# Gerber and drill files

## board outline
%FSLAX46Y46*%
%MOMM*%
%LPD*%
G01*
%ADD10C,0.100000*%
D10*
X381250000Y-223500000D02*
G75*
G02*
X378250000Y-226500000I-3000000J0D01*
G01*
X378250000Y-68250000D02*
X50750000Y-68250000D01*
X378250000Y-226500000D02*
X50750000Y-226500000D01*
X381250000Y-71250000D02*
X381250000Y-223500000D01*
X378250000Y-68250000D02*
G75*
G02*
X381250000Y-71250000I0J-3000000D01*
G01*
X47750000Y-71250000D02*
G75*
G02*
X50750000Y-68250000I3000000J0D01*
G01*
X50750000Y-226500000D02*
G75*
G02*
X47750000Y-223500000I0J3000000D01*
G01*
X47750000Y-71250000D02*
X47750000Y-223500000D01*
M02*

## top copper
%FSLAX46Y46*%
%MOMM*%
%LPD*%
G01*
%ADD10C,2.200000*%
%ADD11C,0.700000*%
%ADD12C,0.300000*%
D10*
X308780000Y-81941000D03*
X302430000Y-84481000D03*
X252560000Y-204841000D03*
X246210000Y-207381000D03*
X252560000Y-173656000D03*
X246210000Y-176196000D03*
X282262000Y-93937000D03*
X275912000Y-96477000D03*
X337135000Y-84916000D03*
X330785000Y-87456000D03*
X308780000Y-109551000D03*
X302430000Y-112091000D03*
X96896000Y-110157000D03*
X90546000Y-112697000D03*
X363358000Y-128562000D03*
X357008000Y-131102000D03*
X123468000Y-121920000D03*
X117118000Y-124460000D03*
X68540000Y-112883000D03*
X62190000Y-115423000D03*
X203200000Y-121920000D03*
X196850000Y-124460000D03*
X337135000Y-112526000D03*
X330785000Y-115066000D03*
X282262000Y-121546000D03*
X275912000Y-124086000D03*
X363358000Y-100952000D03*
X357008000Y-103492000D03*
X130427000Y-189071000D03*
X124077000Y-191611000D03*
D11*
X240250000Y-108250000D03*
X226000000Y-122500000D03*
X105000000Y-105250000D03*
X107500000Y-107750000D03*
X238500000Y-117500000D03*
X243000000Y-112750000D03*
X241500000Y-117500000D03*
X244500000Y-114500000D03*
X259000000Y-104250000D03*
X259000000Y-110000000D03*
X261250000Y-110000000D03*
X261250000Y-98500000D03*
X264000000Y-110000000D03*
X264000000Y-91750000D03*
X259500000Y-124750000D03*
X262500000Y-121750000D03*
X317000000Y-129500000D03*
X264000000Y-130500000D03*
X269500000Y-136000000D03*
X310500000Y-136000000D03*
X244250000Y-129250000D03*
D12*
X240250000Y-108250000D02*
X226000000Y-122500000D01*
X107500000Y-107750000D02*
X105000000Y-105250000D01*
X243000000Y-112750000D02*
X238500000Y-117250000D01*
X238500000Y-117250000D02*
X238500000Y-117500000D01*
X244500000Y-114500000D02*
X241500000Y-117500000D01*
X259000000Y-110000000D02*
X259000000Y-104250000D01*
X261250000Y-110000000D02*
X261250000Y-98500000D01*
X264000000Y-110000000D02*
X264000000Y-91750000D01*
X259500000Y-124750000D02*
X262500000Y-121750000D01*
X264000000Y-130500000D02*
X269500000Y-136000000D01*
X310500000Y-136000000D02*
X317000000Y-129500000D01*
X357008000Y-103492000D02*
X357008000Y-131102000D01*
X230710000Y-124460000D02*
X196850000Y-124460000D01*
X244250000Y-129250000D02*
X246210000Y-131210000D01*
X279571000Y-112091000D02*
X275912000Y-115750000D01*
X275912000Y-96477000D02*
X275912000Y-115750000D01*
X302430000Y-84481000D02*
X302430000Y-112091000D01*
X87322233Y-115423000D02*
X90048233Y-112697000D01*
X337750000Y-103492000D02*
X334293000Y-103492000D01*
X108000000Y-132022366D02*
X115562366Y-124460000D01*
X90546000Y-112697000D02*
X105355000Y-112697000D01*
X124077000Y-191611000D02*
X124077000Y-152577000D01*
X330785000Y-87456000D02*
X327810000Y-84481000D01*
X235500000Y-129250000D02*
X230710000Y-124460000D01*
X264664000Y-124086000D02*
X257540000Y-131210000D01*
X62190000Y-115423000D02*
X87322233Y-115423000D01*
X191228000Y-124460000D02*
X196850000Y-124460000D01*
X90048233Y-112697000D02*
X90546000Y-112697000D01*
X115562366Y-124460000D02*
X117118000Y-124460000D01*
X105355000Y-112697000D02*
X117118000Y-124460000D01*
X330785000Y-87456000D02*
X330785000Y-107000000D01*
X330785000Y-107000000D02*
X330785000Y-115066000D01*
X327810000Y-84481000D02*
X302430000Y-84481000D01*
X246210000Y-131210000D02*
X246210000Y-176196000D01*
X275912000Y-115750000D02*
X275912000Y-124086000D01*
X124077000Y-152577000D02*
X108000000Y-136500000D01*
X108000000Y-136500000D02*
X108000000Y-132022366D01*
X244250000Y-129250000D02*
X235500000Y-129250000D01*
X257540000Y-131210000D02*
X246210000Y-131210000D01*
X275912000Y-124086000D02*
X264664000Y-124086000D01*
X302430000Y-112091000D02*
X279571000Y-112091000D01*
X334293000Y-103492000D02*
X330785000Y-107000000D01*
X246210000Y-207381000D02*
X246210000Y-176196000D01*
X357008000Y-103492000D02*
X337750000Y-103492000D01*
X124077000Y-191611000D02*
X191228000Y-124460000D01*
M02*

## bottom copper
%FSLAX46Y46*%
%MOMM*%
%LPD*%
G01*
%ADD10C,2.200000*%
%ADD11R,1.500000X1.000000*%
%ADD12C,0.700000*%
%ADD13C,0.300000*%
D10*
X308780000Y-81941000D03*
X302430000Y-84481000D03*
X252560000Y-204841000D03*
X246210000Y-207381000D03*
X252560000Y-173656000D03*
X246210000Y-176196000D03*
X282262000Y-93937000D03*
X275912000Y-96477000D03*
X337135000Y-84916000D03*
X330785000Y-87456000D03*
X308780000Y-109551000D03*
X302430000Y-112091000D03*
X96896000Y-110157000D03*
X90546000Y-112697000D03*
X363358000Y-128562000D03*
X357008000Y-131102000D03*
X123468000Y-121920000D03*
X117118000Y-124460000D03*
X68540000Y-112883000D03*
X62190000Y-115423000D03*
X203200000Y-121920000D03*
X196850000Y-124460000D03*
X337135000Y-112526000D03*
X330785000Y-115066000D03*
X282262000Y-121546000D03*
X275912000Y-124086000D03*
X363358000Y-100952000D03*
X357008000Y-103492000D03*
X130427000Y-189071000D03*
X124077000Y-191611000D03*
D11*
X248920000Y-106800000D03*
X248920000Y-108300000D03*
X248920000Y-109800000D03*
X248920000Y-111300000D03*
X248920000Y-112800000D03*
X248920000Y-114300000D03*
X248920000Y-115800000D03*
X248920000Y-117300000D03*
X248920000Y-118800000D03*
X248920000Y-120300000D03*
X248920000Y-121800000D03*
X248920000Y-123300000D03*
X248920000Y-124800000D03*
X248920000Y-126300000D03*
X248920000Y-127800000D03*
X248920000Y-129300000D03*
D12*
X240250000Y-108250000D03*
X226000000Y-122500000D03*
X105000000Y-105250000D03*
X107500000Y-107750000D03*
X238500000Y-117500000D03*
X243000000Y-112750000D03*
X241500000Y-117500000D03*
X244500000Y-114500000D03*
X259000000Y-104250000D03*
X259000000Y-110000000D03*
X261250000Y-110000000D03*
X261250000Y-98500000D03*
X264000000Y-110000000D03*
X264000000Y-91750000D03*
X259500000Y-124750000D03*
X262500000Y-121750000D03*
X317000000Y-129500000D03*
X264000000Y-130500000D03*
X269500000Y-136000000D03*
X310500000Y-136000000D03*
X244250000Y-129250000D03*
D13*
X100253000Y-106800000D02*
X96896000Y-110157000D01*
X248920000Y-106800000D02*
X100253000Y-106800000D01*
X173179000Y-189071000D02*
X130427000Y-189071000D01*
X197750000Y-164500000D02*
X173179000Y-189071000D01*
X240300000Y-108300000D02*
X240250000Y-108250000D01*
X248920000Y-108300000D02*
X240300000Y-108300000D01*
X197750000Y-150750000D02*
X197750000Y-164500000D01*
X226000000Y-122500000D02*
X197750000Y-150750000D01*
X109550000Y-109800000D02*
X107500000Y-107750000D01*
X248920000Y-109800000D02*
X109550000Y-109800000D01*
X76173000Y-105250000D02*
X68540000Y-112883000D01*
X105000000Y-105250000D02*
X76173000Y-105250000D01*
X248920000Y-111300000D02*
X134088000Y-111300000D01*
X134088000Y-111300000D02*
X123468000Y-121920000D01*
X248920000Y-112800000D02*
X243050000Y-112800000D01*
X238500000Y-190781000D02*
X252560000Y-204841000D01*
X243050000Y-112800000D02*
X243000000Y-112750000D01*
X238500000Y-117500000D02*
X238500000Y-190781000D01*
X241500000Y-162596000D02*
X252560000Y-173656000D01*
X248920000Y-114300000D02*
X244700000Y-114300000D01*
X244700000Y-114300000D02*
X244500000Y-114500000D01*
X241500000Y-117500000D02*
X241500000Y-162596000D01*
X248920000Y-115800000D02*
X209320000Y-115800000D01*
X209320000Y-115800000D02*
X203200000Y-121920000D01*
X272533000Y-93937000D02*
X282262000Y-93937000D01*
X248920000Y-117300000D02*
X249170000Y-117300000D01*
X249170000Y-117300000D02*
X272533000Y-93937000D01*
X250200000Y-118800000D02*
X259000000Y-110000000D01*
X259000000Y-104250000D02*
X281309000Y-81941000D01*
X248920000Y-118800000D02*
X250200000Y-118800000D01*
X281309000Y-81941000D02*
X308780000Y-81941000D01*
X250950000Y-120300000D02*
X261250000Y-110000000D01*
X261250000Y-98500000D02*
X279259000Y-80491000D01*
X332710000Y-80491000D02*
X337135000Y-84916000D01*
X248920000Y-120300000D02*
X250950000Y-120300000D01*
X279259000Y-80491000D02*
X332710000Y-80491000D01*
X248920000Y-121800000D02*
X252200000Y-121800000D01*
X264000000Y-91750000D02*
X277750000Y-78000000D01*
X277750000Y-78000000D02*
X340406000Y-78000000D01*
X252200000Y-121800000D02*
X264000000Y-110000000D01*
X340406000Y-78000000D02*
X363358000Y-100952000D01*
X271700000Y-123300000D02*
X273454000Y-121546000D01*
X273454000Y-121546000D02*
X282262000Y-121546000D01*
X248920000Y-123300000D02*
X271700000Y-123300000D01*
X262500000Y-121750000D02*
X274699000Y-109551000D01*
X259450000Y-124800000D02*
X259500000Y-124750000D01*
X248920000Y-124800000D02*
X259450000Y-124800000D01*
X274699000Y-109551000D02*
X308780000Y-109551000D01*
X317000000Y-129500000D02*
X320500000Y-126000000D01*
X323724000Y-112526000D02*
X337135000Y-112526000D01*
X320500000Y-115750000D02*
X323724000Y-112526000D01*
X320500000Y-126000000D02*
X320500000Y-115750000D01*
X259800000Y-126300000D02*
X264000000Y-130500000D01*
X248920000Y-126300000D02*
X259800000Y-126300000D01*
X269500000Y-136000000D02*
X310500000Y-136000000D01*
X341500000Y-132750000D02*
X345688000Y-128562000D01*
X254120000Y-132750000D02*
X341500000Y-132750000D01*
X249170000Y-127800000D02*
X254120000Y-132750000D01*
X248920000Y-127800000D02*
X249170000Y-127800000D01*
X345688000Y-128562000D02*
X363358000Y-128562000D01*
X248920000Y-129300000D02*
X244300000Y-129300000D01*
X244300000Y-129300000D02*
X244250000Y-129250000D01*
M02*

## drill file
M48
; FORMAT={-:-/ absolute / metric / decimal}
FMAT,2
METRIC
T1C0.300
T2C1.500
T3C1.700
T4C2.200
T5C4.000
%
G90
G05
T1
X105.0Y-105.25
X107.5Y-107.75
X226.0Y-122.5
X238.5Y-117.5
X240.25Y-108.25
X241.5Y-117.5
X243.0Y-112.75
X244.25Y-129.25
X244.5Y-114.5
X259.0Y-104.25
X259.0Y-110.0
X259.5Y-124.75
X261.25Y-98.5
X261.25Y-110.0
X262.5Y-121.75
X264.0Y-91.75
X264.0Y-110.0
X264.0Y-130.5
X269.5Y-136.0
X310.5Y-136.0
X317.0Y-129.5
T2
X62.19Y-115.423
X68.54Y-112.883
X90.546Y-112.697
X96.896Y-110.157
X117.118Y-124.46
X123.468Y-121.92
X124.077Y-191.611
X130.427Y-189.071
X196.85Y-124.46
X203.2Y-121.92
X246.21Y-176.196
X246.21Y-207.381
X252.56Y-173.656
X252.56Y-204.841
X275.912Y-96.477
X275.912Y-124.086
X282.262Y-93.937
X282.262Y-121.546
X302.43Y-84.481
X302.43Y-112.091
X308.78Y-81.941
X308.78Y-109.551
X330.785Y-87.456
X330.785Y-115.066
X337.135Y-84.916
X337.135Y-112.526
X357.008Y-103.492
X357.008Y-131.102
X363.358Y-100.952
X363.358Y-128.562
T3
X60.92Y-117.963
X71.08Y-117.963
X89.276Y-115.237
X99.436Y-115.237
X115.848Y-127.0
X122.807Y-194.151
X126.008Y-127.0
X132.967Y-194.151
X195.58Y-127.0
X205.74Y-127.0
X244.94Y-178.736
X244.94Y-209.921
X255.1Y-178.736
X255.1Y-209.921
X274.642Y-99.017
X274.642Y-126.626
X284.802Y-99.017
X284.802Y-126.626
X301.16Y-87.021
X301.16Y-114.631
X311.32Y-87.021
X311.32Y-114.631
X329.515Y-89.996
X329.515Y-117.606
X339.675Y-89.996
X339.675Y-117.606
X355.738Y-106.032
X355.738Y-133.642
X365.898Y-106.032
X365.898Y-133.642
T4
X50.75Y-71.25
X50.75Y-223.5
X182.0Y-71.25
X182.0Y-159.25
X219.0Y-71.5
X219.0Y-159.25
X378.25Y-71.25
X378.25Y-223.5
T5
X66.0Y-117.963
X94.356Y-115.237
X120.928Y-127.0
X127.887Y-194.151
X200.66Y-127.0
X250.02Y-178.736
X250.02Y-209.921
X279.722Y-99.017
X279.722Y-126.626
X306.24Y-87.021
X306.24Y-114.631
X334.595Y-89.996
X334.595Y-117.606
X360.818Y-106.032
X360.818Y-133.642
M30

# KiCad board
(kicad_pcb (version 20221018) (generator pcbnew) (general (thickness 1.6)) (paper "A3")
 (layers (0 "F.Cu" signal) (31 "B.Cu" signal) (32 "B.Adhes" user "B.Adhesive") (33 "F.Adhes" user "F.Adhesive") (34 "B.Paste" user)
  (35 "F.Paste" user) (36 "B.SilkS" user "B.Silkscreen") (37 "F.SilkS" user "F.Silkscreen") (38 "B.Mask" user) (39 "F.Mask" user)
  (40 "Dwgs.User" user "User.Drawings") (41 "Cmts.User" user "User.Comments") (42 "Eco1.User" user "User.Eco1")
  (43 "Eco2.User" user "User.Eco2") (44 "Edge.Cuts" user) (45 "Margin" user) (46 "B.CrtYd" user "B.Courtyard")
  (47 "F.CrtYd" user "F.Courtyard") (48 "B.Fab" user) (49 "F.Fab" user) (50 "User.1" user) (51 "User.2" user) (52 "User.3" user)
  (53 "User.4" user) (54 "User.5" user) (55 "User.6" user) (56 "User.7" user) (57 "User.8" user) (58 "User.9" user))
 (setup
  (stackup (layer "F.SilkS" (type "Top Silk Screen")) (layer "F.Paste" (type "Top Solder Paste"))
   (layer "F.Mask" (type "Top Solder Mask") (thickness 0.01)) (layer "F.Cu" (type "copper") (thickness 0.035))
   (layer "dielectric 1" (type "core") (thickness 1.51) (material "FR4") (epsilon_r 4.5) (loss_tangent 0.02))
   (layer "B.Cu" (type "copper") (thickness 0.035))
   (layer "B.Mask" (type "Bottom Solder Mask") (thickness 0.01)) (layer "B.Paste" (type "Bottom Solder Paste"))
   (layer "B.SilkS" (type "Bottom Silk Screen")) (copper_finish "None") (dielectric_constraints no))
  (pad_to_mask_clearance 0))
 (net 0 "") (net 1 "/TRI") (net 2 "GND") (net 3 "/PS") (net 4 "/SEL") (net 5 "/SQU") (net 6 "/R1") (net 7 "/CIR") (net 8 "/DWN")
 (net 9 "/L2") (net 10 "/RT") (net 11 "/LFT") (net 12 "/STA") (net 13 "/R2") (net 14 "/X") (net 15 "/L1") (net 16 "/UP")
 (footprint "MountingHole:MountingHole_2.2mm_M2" (layer "F.Cu") (at 50.75 223.5)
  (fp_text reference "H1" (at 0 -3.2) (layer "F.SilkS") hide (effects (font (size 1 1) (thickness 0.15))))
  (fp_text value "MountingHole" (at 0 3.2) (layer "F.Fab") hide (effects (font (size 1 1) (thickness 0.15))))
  (pad "" np_thru_hole circle (at 0 0) (size 2.2 2.2) (drill 2.2) (layers "*.Cu" "*.Mask")))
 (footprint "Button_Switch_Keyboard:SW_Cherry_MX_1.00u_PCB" (layer "F.Cu") (at 308.78 81.941)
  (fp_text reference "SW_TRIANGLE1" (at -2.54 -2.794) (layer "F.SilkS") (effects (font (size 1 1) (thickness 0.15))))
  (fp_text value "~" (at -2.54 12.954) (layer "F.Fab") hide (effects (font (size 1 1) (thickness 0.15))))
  (pad "" np_thru_hole circle (at -7.62 5.08) (size 1.7 1.7) (drill 1.7) (layers "*.Cu" "*.Mask"))
  (pad "" np_thru_hole circle (at -2.54 5.08) (size 4 4) (drill 4) (layers "*.Cu" "*.Mask"))
  (pad "" np_thru_hole circle (at 2.54 5.08) (size 1.7 1.7) (drill 1.7) (layers "*.Cu" "*.Mask"))
  (pad "1" thru_hole circle (at 0 0) (size 2.2 2.2) (drill 1.5) (layers "*.Cu" "*.Mask") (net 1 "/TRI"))
  (pad "2" thru_hole circle (at -6.35 2.54) (size 2.2 2.2) (drill 1.5) (layers "*.Cu" "*.Mask") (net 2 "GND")))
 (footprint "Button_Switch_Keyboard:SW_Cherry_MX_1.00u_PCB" (layer "F.Cu") (at 252.56 204.841)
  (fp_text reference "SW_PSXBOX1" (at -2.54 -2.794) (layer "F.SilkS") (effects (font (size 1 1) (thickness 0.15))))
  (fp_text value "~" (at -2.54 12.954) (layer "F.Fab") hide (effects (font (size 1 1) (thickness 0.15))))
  (pad "" np_thru_hole circle (at -7.62 5.08) (size 1.7 1.7) (drill 1.7) (layers "*.Cu" "*.Mask"))
  (pad "" np_thru_hole circle (at -2.54 5.08) (size 4 4) (drill 4) (layers "*.Cu" "*.Mask"))
  (pad "" np_thru_hole circle (at 2.54 5.08) (size 1.7 1.7) (drill 1.7) (layers "*.Cu" "*.Mask"))
  (pad "1" thru_hole circle (at 0 0) (size 2.2 2.2) (drill 1.5) (layers "*.Cu" "*.Mask") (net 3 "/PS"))
  (pad "2" thru_hole circle (at -6.35 2.54) (size 2.2 2.2) (drill 1.5) (layers "*.Cu" "*.Mask") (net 2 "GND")))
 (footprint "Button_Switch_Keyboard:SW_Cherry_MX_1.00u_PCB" (layer "F.Cu") (at 252.56 173.656)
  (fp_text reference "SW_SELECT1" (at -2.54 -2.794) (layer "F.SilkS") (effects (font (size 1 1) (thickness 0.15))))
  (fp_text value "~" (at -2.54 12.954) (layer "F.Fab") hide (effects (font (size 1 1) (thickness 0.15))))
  (pad "" np_thru_hole circle (at -7.62 5.08) (size 1.7 1.7) (drill 1.7) (layers "*.Cu" "*.Mask"))
  (pad "" np_thru_hole circle (at -2.54 5.08) (size 4 4) (drill 4) (layers "*.Cu" "*.Mask"))
  (pad "" np_thru_hole circle (at 2.54 5.08) (size 1.7 1.7) (drill 1.7) (layers "*.Cu" "*.Mask"))
  (pad "1" thru_hole circle (at 0 0) (size 2.2 2.2) (drill 1.5) (layers "*.Cu" "*.Mask") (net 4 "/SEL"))
  (pad "2" thru_hole circle (at -6.35 2.54) (size 2.2 2.2) (drill 1.5) (layers "*.Cu" "*.Mask") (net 2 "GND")))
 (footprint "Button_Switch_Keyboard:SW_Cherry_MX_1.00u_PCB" (layer "F.Cu") (at 282.262 93.937)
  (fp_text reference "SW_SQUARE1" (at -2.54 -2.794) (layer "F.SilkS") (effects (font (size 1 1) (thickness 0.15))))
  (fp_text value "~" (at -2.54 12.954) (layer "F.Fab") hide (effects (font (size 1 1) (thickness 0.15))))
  (pad "" np_thru_hole circle (at -7.62 5.08) (size 1.7 1.7) (drill 1.7) (layers "*.Cu" "*.Mask"))
  (pad "" np_thru_hole circle (at -2.54 5.08) (size 4 4) (drill 4) (layers "*.Cu" "*.Mask"))
  (pad "" np_thru_hole circle (at 2.54 5.08) (size 1.7 1.7) (drill 1.7) (layers "*.Cu" "*.Mask"))
  (pad "1" thru_hole circle (at 0 0) (size 2.2 2.2) (drill 1.5) (layers "*.Cu" "*.Mask") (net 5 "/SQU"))
  (pad "2" thru_hole circle (at -6.35 2.54) (size 2.2 2.2) (drill 1.5) (layers "*.Cu" "*.Mask") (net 2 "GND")))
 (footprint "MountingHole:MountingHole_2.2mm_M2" (layer "F.Cu") (at 50.75 71.25)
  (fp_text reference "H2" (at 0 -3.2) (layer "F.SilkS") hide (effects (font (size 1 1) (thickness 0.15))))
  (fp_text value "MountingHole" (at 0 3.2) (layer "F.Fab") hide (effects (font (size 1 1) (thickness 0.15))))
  (pad "" np_thru_hole circle (at 0 0) (size 2.2 2.2) (drill 2.2) (layers "*.Cu" "*.Mask")))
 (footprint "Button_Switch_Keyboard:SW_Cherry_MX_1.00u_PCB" (layer "F.Cu") (at 337.135 84.916)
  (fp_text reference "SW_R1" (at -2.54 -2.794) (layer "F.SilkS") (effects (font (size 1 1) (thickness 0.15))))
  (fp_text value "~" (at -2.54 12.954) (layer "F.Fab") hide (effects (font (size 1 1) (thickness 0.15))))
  (pad "" np_thru_hole circle (at -7.62 5.08) (size 1.7 1.7) (drill 1.7) (layers "*.Cu" "*.Mask"))
  (pad "" np_thru_hole circle (at -2.54 5.08) (size 4 4) (drill 4) (layers "*.Cu" "*.Mask"))
  (pad "" np_thru_hole circle (at 2.54 5.08) (size 1.7 1.7) (drill 1.7) (layers "*.Cu" "*.Mask"))
  (pad "1" thru_hole circle (at 0 0) (size 2.2 2.2) (drill 1.5) (layers "*.Cu" "*.Mask") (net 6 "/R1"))
  (pad "2" thru_hole circle (at -6.35 2.54) (size 2.2 2.2) (drill 1.5) (layers "*.Cu" "*.Mask") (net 2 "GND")))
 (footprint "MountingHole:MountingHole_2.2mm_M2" (layer "F.Cu") (at 219 71.5)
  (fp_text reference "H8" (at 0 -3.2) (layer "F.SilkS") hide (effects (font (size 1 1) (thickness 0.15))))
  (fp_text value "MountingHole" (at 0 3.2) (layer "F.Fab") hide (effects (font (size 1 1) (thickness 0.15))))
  (pad "" np_thru_hole circle (at 0 0) (size 2.2 2.2) (drill 2.2) (layers "*.Cu" "*.Mask")))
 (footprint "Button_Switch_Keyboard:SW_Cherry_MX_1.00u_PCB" (layer "F.Cu") (at 308.78 109.551)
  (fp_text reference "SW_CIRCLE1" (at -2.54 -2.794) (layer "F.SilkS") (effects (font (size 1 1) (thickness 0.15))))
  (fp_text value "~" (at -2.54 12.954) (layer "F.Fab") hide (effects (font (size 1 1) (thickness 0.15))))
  (pad "" np_thru_hole circle (at -7.62 5.08) (size 1.7 1.7) (drill 1.7) (layers "*.Cu" "*.Mask"))
  (pad "" np_thru_hole circle (at -2.54 5.08) (size 4 4) (drill 4) (layers "*.Cu" "*.Mask"))
  (pad "" np_thru_hole circle (at 2.54 5.08) (size 1.7 1.7) (drill 1.7) (layers "*.Cu" "*.Mask"))
  (pad "1" thru_hole circle (at 0 0) (size 2.2 2.2) (drill 1.5) (layers "*.Cu" "*.Mask") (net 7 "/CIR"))
  (pad "2" thru_hole circle (at -6.35 2.54) (size 2.2 2.2) (drill 1.5) (layers "*.Cu" "*.Mask") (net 2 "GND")))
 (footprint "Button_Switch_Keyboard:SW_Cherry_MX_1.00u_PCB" (layer "F.Cu") (at 96.896 110.157)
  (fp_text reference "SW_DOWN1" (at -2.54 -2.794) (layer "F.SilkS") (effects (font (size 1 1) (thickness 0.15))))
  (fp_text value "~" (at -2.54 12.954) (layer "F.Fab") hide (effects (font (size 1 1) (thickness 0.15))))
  (pad "" np_thru_hole circle (at -7.62 5.08) (size 1.7 1.7) (drill 1.7) (layers "*.Cu" "*.Mask"))
  (pad "" np_thru_hole circle (at -2.54 5.08) (size 4 4) (drill 4) (layers "*.Cu" "*.Mask"))
  (pad "" np_thru_hole circle (at 2.54 5.08) (size 1.7 1.7) (drill 1.7) (layers "*.Cu" "*.Mask"))
  (pad "1" thru_hole circle (at 0 0) (size 2.2 2.2) (drill 1.5) (layers "*.Cu" "*.Mask") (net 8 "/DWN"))
  (pad "2" thru_hole circle (at -6.35 2.54) (size 2.2 2.2) (drill 1.5) (layers "*.Cu" "*.Mask") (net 2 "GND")))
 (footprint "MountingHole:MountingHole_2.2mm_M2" (layer "F.Cu") (at 219 159.25)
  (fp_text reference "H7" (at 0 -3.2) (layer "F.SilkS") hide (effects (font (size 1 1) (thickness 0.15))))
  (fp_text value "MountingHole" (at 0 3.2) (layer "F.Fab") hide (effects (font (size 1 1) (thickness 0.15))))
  (pad "" np_thru_hole circle (at 0 0) (size 2.2 2.2) (drill 2.2) (layers "*.Cu" "*.Mask")))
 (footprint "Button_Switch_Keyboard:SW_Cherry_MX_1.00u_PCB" (layer "F.Cu") (at 363.358 128.562)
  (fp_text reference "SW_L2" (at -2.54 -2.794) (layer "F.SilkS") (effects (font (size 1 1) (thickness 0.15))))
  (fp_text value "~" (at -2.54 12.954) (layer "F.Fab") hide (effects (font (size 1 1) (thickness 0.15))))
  (pad "" np_thru_hole circle (at -7.62 5.08) (size 1.7 1.7) (drill 1.7) (layers "*.Cu" "*.Mask"))
  (pad "" np_thru_hole circle (at -2.54 5.08) (size 4 4) (drill 4) (layers "*.Cu" "*.Mask"))
  (pad "" np_thru_hole circle (at 2.54 5.08) (size 1.7 1.7) (drill 1.7) (layers "*.Cu" "*.Mask"))
  (pad "1" thru_hole circle (at 0 0) (size 2.2 2.2) (drill 1.5) (layers "*.Cu" "*.Mask") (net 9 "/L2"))
  (pad "2" thru_hole circle (at -6.35 2.54) (size 2.2 2.2) (drill 1.5) (layers "*.Cu" "*.Mask") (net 2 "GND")))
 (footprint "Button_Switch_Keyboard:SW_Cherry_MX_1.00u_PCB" (layer "F.Cu") (at 123.468 121.92)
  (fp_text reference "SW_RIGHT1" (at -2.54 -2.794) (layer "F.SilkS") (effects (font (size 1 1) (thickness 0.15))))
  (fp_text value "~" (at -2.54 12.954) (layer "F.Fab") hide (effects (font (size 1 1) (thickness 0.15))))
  (pad "" np_thru_hole circle (at -7.62 5.08) (size 1.7 1.7) (drill 1.7) (layers "*.Cu" "*.Mask"))
  (pad "" np_thru_hole circle (at -2.54 5.08) (size 4 4) (drill 4) (layers "*.Cu" "*.Mask"))
  (pad "" np_thru_hole circle (at 2.54 5.08) (size 1.7 1.7) (drill 1.7) (layers "*.Cu" "*.Mask"))
  (pad "1" thru_hole circle (at 0 0) (size 2.2 2.2) (drill 1.5) (layers "*.Cu" "*.Mask") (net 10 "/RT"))
  (pad "2" thru_hole circle (at -6.35 2.54) (size 2.2 2.2) (drill 1.5) (layers "*.Cu" "*.Mask") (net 2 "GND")))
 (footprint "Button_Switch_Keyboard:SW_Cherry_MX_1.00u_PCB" (layer "F.Cu") (at 68.54 112.883)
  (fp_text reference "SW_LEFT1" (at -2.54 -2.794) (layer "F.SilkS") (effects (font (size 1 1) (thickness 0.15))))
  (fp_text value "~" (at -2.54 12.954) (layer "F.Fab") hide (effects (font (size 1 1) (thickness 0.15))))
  (pad "" np_thru_hole circle (at -7.62 5.08) (size 1.7 1.7) (drill 1.7) (layers "*.Cu" "*.Mask"))
  (pad "" np_thru_hole circle (at -2.54 5.08) (size 4 4) (drill 4) (layers "*.Cu" "*.Mask"))
  (pad "" np_thru_hole circle (at 2.54 5.08) (size 1.7 1.7) (drill 1.7) (layers "*.Cu" "*.Mask"))
  (pad "1" thru_hole circle (at 0 0) (size 2.2 2.2) (drill 1.5) (layers "*.Cu" "*.Mask") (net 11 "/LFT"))
  (pad "2" thru_hole circle (at -6.35 2.54) (size 2.2 2.2) (drill 1.5) (layers "*.Cu" "*.Mask") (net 2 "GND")))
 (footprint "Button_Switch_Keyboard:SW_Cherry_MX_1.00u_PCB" (layer "F.Cu") (at 203.2 121.92)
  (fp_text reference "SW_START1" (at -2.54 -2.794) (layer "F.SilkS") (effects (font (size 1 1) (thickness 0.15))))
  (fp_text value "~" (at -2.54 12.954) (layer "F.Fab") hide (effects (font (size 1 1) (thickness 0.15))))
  (pad "" np_thru_hole circle (at -7.62 5.08) (size 1.7 1.7) (drill 1.7) (layers "*.Cu" "*.Mask"))
  (pad "" np_thru_hole circle (at -2.54 5.08) (size 4 4) (drill 4) (layers "*.Cu" "*.Mask"))
  (pad "" np_thru_hole circle (at 2.54 5.08) (size 1.7 1.7) (drill 1.7) (layers "*.Cu" "*.Mask"))
  (pad "1" thru_hole circle (at 0 0) (size 2.2 2.2) (drill 1.5) (layers "*.Cu" "*.Mask") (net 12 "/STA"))
  (pad "2" thru_hole circle (at -6.35 2.54) (size 2.2 2.2) (drill 1.5) (layers "*.Cu" "*.Mask") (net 2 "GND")))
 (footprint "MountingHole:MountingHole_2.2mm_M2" (layer "F.Cu") (at 182 71.25)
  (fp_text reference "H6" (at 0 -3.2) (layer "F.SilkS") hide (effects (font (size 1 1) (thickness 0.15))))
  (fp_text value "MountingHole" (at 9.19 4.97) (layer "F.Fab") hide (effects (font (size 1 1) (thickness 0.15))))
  (pad "" np_thru_hole circle (at 0 0) (size 2.2 2.2) (drill 2.2) (layers "*.Cu" "*.Mask")))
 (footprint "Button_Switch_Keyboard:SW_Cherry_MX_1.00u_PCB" (layer "F.Cu") (at 337.135 112.526)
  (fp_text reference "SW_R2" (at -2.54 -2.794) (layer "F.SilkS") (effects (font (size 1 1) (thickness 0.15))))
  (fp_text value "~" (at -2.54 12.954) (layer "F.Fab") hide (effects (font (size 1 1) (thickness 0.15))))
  (pad "" np_thru_hole circle (at -7.62 5.08) (size 1.7 1.7) (drill 1.7) (layers "*.Cu" "*.Mask"))
  (pad "" np_thru_hole circle (at -2.54 5.08) (size 4 4) (drill 4) (layers "*.Cu" "*.Mask"))
  (pad "" np_thru_hole circle (at 2.54 5.08) (size 1.7 1.7) (drill 1.7) (layers "*.Cu" "*.Mask"))
  (pad "1" thru_hole circle (at 0 0) (size 2.2 2.2) (drill 1.5) (layers "*.Cu" "*.Mask") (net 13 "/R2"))
  (pad "2" thru_hole circle (at -6.35 2.54) (size 2.2 2.2) (drill 1.5) (layers "*.Cu" "*.Mask") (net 2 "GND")))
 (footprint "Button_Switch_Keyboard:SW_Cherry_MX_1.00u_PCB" (layer "F.Cu") (at 282.262 121.546)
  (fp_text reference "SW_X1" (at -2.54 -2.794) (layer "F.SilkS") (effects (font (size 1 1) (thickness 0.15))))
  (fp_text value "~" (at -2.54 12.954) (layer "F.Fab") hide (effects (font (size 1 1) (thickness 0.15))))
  (pad "" np_thru_hole circle (at -7.62 5.08) (size 1.7 1.7) (drill 1.7) (layers "*.Cu" "*.Mask"))
  (pad "" np_thru_hole circle (at -2.54 5.08) (size 4 4) (drill 4) (layers "*.Cu" "*.Mask"))
  (pad "" np_thru_hole circle (at 2.54 5.08) (size 1.7 1.7) (drill 1.7) (layers "*.Cu" "*.Mask"))
  (pad "1" thru_hole circle (at 0 0) (size 2.2 2.2) (drill 1.5) (layers "*.Cu" "*.Mask") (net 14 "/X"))
  (pad "2" thru_hole circle (at -6.35 2.54) (size 2.2 2.2) (drill 1.5) (layers "*.Cu" "*.Mask") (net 2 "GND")))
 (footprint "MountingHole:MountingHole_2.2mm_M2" (layer "F.Cu") (at 378.25 71.25)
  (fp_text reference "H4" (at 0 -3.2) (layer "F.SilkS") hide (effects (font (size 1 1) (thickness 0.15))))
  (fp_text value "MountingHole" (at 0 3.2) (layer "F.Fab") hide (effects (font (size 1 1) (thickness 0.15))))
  (pad "" np_thru_hole circle (at 0 0) (size 2.2 2.2) (drill 2.2) (layers "*.Cu" "*.Mask")))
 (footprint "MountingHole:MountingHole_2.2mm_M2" (layer "F.Cu") (at 378.25 223.5)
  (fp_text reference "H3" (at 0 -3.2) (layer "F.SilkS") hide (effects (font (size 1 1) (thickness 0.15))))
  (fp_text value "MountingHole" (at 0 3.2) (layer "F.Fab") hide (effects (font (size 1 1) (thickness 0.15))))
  (pad "" np_thru_hole circle (at 0 0) (size 2.2 2.2) (drill 2.2) (layers "*.Cu" "*.Mask")))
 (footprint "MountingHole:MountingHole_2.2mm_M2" (layer "F.Cu") (at 182 159.25)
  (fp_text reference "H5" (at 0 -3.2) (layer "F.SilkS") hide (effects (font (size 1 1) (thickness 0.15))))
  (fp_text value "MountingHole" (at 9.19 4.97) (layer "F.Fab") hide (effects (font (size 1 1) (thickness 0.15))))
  (pad "" np_thru_hole circle (at 0 0) (size 2.2 2.2) (drill 2.2) (layers "*.Cu" "*.Mask")))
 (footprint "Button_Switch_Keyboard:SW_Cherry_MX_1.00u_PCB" (layer "F.Cu") (at 363.358 100.952)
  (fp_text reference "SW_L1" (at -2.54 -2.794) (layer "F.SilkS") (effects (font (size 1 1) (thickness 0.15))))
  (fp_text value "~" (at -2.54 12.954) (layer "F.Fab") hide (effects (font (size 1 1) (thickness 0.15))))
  (pad "" np_thru_hole circle (at -7.62 5.08) (size 1.7 1.7) (drill 1.7) (layers "*.Cu" "*.Mask"))
  (pad "" np_thru_hole circle (at -2.54 5.08) (size 4 4) (drill 4) (layers "*.Cu" "*.Mask"))
  (pad "" np_thru_hole circle (at 2.54 5.08) (size 1.7 1.7) (drill 1.7) (layers "*.Cu" "*.Mask"))
  (pad "1" thru_hole circle (at 0 0) (size 2.2 2.2) (drill 1.5) (layers "*.Cu" "*.Mask") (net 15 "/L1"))
  (pad "2" thru_hole circle (at -6.35 2.54) (size 2.2 2.2) (drill 1.5) (layers "*.Cu" "*.Mask") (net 2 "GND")))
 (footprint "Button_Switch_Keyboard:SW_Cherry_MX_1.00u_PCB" (layer "F.Cu") (at 130.427 189.071)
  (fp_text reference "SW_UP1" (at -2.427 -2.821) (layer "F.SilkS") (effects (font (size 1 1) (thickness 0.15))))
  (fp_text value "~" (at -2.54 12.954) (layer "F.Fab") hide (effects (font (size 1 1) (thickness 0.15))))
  (pad "" np_thru_hole circle (at -7.62 5.08) (size 1.7 1.7) (drill 1.7) (layers "*.Cu" "*.Mask"))
  (pad "" np_thru_hole circle (at -2.54 5.08) (size 4 4) (drill 4) (layers "*.Cu" "*.Mask"))
  (pad "" np_thru_hole circle (at 2.54 5.08) (size 1.7 1.7) (drill 1.7) (layers "*.Cu" "*.Mask"))
  (pad "1" thru_hole circle (at 0 0) (size 2.2 2.2) (drill 1.5) (layers "*.Cu" "*.Mask") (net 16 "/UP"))
  (pad "2" thru_hole circle (at -6.35 2.54) (size 2.2 2.2) (drill 1.5) (layers "*.Cu" "*.Mask") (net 2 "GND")))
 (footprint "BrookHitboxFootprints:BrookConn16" (layer "B.Cu") (at 248.92 118.05 -90)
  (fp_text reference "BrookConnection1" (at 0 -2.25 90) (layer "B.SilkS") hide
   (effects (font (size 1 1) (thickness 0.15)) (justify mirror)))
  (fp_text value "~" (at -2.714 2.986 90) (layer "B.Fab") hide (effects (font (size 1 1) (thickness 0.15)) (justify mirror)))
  (pad "1" smd rect (at -11.25 0 270) (size 1 1.5) (layers "B.Cu" "B.Paste" "B.Mask") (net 8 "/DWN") (thermal_bridge_angle 45))
  (pad "2" smd rect (at -9.75 0 270) (size 1 1.5) (layers "B.Cu" "B.Paste" "B.Mask") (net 16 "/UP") (thermal_bridge_angle 45))
  (pad "3" smd rect (at -8.25 0 270) (size 1 1.5) (layers "B.Cu" "B.Paste" "B.Mask") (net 11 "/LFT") (thermal_bridge_angle 45))
  (pad "4" smd rect (at -6.75 0 270) (size 1 1.5) (layers "B.Cu" "B.Paste" "B.Mask") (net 10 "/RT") (thermal_bridge_angle 45))
  (pad "5" smd rect (at -5.25 0 270) (size 1 1.5) (layers "B.Cu" "B.Paste" "B.Mask") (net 3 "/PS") (thermal_bridge_angle 45))
  (pad "6" smd rect (at -3.75 0 270) (size 1 1.5) (layers "B.Cu" "B.Paste" "B.Mask") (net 4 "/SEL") (thermal_bridge_angle 45))
  (pad "7" smd rect (at -2.25 0 270) (size 1 1.5) (layers "B.Cu" "B.Paste" "B.Mask") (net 12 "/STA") (thermal_bridge_angle 45))
  (pad "8" smd rect (at -0.75 0 270) (size 1 1.5) (layers "B.Cu" "B.Paste" "B.Mask") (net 5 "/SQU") (thermal_bridge_angle 45))
  (pad "9" smd rect (at 0.75 0 270) (size 1 1.5) (layers "B.Cu" "B.Paste" "B.Mask") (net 1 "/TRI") (thermal_bridge_angle 45))
  (pad "10" smd rect (at 2.25 0 270) (size 1 1.5) (layers "B.Cu" "B.Paste" "B.Mask") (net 6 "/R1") (thermal_bridge_angle 45))
  (pad "11" smd rect (at 3.75 0 270) (size 1 1.5) (layers "B.Cu" "B.Paste" "B.Mask") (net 15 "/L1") (thermal_bridge_angle 45))
  (pad "12" smd rect (at 5.25 0 270) (size 1 1.5) (layers "B.Cu" "B.Paste" "B.Mask") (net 14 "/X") (thermal_bridge_angle 45))
  (pad "13" smd rect (at 6.75 0 270) (size 1 1.5) (layers "B.Cu" "B.Paste" "B.Mask") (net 7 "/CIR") (thermal_bridge_angle 45))
  (pad "14" smd rect (at 8.25 0 270) (size 1 1.5) (layers "B.Cu" "B.Paste" "B.Mask") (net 13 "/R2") (thermal_bridge_angle 45))
  (pad "15" smd rect (at 9.75 0 270) (size 1 1.5) (layers "B.Cu" "B.Paste" "B.Mask") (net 9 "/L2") (thermal_bridge_angle 45))
  (pad "16" smd rect (at 11.25 0 270) (size 1 1.5) (layers "B.Cu" "B.Paste" "B.Mask") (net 2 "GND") (thermal_bridge_angle 45)))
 (gr_arc (start 381.25 223.5) (mid 380.37132 225.62132) (end 378.25 226.5) (stroke (width 0.1) (type default)) (layer "Edge.Cuts"))
 (gr_line (start 378.25 68.25) (end 50.75 68.25) (stroke (width 0.1) (type default)) (layer "Edge.Cuts"))
 (gr_line (start 378.25 226.5) (end 50.75 226.5) (stroke (width 0.1) (type default)) (layer "Edge.Cuts"))
 (gr_line (start 381.25 71.25) (end 381.25 223.5) (stroke (width 0.1) (type default)) (layer "Edge.Cuts"))
 (gr_arc (start 378.25 68.25) (mid 380.37132 69.12868) (end 381.25 71.25) (stroke (width 0.1) (type default)) (layer "Edge.Cuts"))
 (gr_arc (start 47.75 71.25) (mid 48.62868 69.12868) (end 50.75 68.25) (stroke (width 0.1) (type default)) (layer "Edge.Cuts"))
 (gr_arc (start 50.75 226.5) (mid 48.62868 225.62132) (end 47.75 223.5) (stroke (width 0.1) (type default)) (layer "Edge.Cuts"))
 (gr_line (start 47.75 71.25) (end 47.75 223.5) (stroke (width 0.1) (type default)) (layer "Edge.Cuts"))
 (segment (start 100.253 106.8) (end 96.896 110.157) (width 0.3) (layer "B.Cu") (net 8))
 (segment (start 248.92 106.8) (end 100.253 106.8) (width 0.3) (layer "B.Cu") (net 8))
 (segment (start 240.25 108.25) (end 226 122.5) (width 0.3) (layer "F.Cu") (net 16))
 (via (at 240.25 108.25) (size 0.7) (drill 0.3) (layers "F.Cu" "B.Cu") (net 16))
 (via (at 226 122.5) (size 0.7) (drill 0.3) (layers "F.Cu" "B.Cu") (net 16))
 (segment (start 173.179 189.071) (end 130.427 189.071) (width 0.3) (layer "B.Cu") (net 16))
 (segment (start 197.75 164.5) (end 173.179 189.071) (width 0.3) (layer "B.Cu") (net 16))
 (segment (start 240.3 108.3) (end 240.25 108.25) (width 0.3) (layer "B.Cu") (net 16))
 (segment (start 248.92 108.3) (end 240.3 108.3) (width 0.3) (layer "B.Cu") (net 16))
 (segment (start 197.75 150.75) (end 197.75 164.5) (width 0.3) (layer "B.Cu") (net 16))
 (segment (start 226 122.5) (end 197.75 150.75) (width 0.3) (layer "B.Cu") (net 16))
 (segment (start 107.5 107.75) (end 105 105.25) (width 0.3) (layer "F.Cu") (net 11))
 (via (at 105 105.25) (size 0.7) (drill 0.3) (layers "F.Cu" "B.Cu") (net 11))
 (via (at 107.5 107.75) (size 0.7) (drill 0.3) (layers "F.Cu" "B.Cu") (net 11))
 (segment (start 109.55 109.8) (end 107.5 107.75) (width 0.3) (layer "B.Cu") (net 11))
 (segment (start 248.92 109.8) (end 109.55 109.8) (width 0.3) (layer "B.Cu") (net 11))
 (segment (start 76.173 105.25) (end 68.54 112.883) (width 0.3) (layer "B.Cu") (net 11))
 (segment (start 105 105.25) (end 76.173 105.25) (width 0.3) (layer "B.Cu") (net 11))
 (segment (start 248.92 111.3) (end 134.088 111.3) (width 0.3) (layer "B.Cu") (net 10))
 (segment (start 134.088 111.3) (end 123.468 121.92) (width 0.3) (layer "B.Cu") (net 10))
 (segment (start 243 112.75) (end 238.5 117.25) (width 0.3) (layer "F.Cu") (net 3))
 (segment (start 238.5 117.25) (end 238.5 117.5) (width 0.3) (layer "F.Cu") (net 3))
 (via (at 238.5 117.5) (size 0.7) (drill 0.3) (layers "F.Cu" "B.Cu") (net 3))
 (via (at 243 112.75) (size 0.7) (drill 0.3) (layers "F.Cu" "B.Cu") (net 3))
 (segment (start 248.92 112.8) (end 243.05 112.8) (width 0.3) (layer "B.Cu") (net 3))
 (segment (start 238.5 190.781) (end 252.56 204.841) (width 0.3) (layer "B.Cu") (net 3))
 (segment (start 243.05 112.8) (end 243 112.75) (width 0.3) (layer "B.Cu") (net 3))
 (segment (start 238.5 117.5) (end 238.5 190.781) (width 0.3) (layer "B.Cu") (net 3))
 (segment (start 244.5 114.5) (end 241.5 117.5) (width 0.3) (layer "F.Cu") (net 4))
 (via (at 241.5 117.5) (size 0.7) (drill 0.3) (layers "F.Cu" "B.Cu") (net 4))
 (via (at 244.5 114.5) (size 0.7) (drill 0.3) (layers "F.Cu" "B.Cu") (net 4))
 (segment (start 241.5 162.596) (end 252.56 173.656) (width 0.3) (layer "B.Cu") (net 4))
 (segment (start 248.92 114.3) (end 244.7 114.3) (width 0.3) (layer "B.Cu") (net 4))
 (segment (start 244.7 114.3) (end 244.5 114.5) (width 0.3) (layer "B.Cu") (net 4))
 (segment (start 241.5 117.5) (end 241.5 162.596) (width 0.3) (layer "B.Cu") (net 4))
 (segment (start 248.92 115.8) (end 209.32 115.8) (width 0.3) (layer "B.Cu") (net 12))
 (segment (start 209.32 115.8) (end 203.2 121.92) (width 0.3) (layer "B.Cu") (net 12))
 (segment (start 272.533 93.937) (end 282.262 93.937) (width 0.3) (layer "B.Cu") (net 5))
 (segment (start 248.92 117.3) (end 249.17 117.3) (width 0.3) (layer "B.Cu") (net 5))
 (segment (start 249.17 117.3) (end 272.533 93.937) (width 0.3) (layer "B.Cu") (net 5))
 (segment (start 259 110) (end 259 104.25) (width 0.3) (layer "F.Cu") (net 1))
 (via (at 259 104.25) (size 0.7) (drill 0.3) (layers "F.Cu" "B.Cu") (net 1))
 (via (at 259 110) (size 0.7) (drill 0.3) (layers "F.Cu" "B.Cu") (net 1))
 (segment (start 250.2 118.8) (end 259 110) (width 0.3) (layer "B.Cu") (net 1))
 (segment (start 259 104.25) (end 281.309 81.941) (width 0.3) (layer "B.Cu") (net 1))
 (segment (start 248.92 118.8) (end 250.2 118.8) (width 0.3) (layer "B.Cu") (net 1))
 (segment (start 281.309 81.941) (end 308.78 81.941) (width 0.3) (layer "B.Cu") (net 1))
 (segment (start 261.25 110) (end 261.25 98.5) (width 0.3) (layer "F.Cu") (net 6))
 (via (at 261.25 110) (size 0.7) (drill 0.3) (layers "F.Cu" "B.Cu") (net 6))
 (via (at 261.25 98.5) (size 0.7) (drill 0.3) (layers "F.Cu" "B.Cu") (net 6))
 (segment (start 250.95 120.3) (end 261.25 110) (width 0.3) (layer "B.Cu") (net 6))
 (segment (start 261.25 98.5) (end 279.259 80.491) (width 0.3) (layer "B.Cu") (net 6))
 (segment (start 332.71 80.491) (end 337.135 84.916) (width 0.3) (layer "B.Cu") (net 6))
 (segment (start 248.92 120.3) (end 250.95 120.3) (width 0.3) (layer "B.Cu") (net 6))
 (segment (start 279.259 80.491) (end 332.71 80.491) (width 0.3) (layer "B.Cu") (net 6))
 (segment (start 264 110) (end 264 91.75) (width 0.3) (layer "F.Cu") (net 15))
 (via (at 264 110) (size 0.7) (drill 0.3) (layers "F.Cu" "B.Cu") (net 15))
 (via (at 264 91.75) (size 0.7) (drill 0.3) (layers "F.Cu" "B.Cu") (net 15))
 (segment (start 248.92 121.8) (end 252.2 121.8) (width 0.3) (layer "B.Cu") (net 15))
 (segment (start 264 91.75) (end 277.75 78) (width 0.3) (layer "B.Cu") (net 15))
 (segment (start 277.75 78) (end 340.406 78) (width 0.3) (layer "B.Cu") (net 15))
 (segment (start 252.2 121.8) (end 264 110) (width 0.3) (layer "B.Cu") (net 15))
 (segment (start 340.406 78) (end 363.358 100.952) (width 0.3) (layer "B.Cu") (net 15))
 (segment (start 271.7 123.3) (end 273.454 121.546) (width 0.3) (layer "B.Cu") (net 14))
 (segment (start 273.454 121.546) (end 282.262 121.546) (width 0.3) (layer "B.Cu") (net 14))
 (segment (start 248.92 123.3) (end 271.7 123.3) (width 0.3) (layer "B.Cu") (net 14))
 (segment (start 259.5 124.75) (end 262.5 121.75) (width 0.3) (layer "F.Cu") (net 7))
 (via (at 259.5 124.75) (size 0.7) (drill 0.3) (layers "F.Cu" "B.Cu") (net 7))
 (via (at 262.5 121.75) (size 0.7) (drill 0.3) (layers "F.Cu" "B.Cu") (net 7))
 (segment (start 262.5 121.75) (end 274.699 109.551) (width 0.3) (layer "B.Cu") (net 7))
 (segment (start 259.45 124.8) (end 259.5 124.75) (width 0.3) (layer "B.Cu") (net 7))
 (segment (start 248.92 124.8) (end 259.45 124.8) (width 0.3) (layer "B.Cu") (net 7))
 (segment (start 274.699 109.551) (end 308.78 109.551) (width 0.3) (layer "B.Cu") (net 7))
 (segment (start 264 130.5) (end 269.5 136) (width 0.3) (layer "F.Cu") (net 13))
 (segment (start 310.5 136) (end 317 129.5) (width 0.3) (layer "F.Cu") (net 13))
 (via (at 317 129.5) (size 0.7) (drill 0.3) (layers "F.Cu" "B.Cu") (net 13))
 (via (at 264 130.5) (size 0.7) (drill 0.3) (layers "F.Cu" "B.Cu") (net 13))
 (via (at 269.5 136) (size 0.7) (drill 0.3) (layers "F.Cu" "B.Cu") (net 13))
 (via (at 310.5 136) (size 0.7) (drill 0.3) (layers "F.Cu" "B.Cu") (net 13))
 (segment (start 317 129.5) (end 320.5 126) (width 0.3) (layer "B.Cu") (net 13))
 (segment (start 323.724 112.526) (end 337.135 112.526) (width 0.3) (layer "B.Cu") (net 13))
 (segment (start 320.5 115.75) (end 323.724 112.526) (width 0.3) (layer "B.Cu") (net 13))
 (segment (start 320.5 126) (end 320.5 115.75) (width 0.3) (layer "B.Cu") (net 13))
 (segment (start 259.8 126.3) (end 264 130.5) (width 0.3) (layer "B.Cu") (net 13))
 (segment (start 248.92 126.3) (end 259.8 126.3) (width 0.3) (layer "B.Cu") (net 13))
 (segment (start 269.5 136) (end 310.5 136) (width 0.3) (layer "B.Cu") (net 13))
 (segment (start 341.5 132.75) (end 345.688 128.562) (width 0.3) (layer "B.Cu") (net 9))
 (segment (start 254.12 132.75) (end 341.5 132.75) (width 0.3) (layer "B.Cu") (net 9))
 (segment (start 249.17 127.8) (end 254.12 132.75) (width 0.3) (layer "B.Cu") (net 9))
 (segment (start 248.92 127.8) (end 249.17 127.8) (width 0.3) (layer "B.Cu") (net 9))
 (segment (start 345.688 128.562) (end 363.358 128.562) (width 0.3) (layer "B.Cu") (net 9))
 (segment (start 357.008 103.492) (end 357.008 131.102) (width 0.3) (layer "F.Cu") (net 2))
 (segment (start 230.71 124.46) (end 196.85 124.46) (width 0.3) (layer "F.Cu") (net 2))
 (segment (start 244.25 129.25) (end 246.21 131.21) (width 0.3) (layer "F.Cu") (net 2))
 (segment (start 279.571 112.091) (end 275.912 115.75) (width 0.3) (layer "F.Cu") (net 2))
 (segment (start 275.912 96.477) (end 275.912 115.75) (width 0.3) (layer "F.Cu") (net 2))
 (segment (start 302.43 84.481) (end 302.43 112.091) (width 0.3) (layer "F.Cu") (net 2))
 (segment (start 87.322233 115.423) (end 90.048233 112.697) (width 0.3) (layer "F.Cu") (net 2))
 (segment (start 337.75 103.492) (end 334.293 103.492) (width 0.3) (layer "F.Cu") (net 2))
 (segment (start 108 132.022366) (end 115.562366 124.46) (width 0.3) (layer "F.Cu") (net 2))
 (segment (start 90.546 112.697) (end 105.355 112.697) (width 0.3) (layer "F.Cu") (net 2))
 (segment (start 124.077 191.611) (end 124.077 152.577) (width 0.3) (layer "F.Cu") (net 2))
 (segment (start 330.785 87.456) (end 327.81 84.481) (width 0.3) (layer "F.Cu") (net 2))
 (segment (start 235.5 129.25) (end 230.71 124.46) (width 0.3) (layer "F.Cu") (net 2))
 (segment (start 264.664 124.086) (end 257.54 131.21) (width 0.3) (layer "F.Cu") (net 2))
 (segment (start 62.19 115.423) (end 87.322233 115.423) (width 0.3) (layer "F.Cu") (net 2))
 (segment (start 191.228 124.46) (end 196.85 124.46) (width 0.3) (layer "F.Cu") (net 2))
 (segment (start 90.048233 112.697) (end 90.546 112.697) (width 0.3) (layer "F.Cu") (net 2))
 (segment (start 115.562366 124.46) (end 117.118 124.46) (width 0.3) (layer "F.Cu") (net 2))
 (segment (start 105.355 112.697) (end 117.118 124.46) (width 0.3) (layer "F.Cu") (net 2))
 (segment (start 330.785 87.456) (end 330.785 107) (width 0.3) (layer "F.Cu") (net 2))
 (segment (start 330.785 107) (end 330.785 115.066) (width 0.3) (layer "F.Cu") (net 2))
 (segment (start 327.81 84.481) (end 302.43 84.481) (width 0.3) (layer "F.Cu") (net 2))
 (segment (start 246.21 131.21) (end 246.21 176.196) (width 0.3) (layer "F.Cu") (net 2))
 (segment (start 275.912 115.75) (end 275.912 124.086) (width 0.3) (layer "F.Cu") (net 2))
 (segment (start 124.077 152.577) (end 108 136.5) (width 0.3) (layer "F.Cu") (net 2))
 (segment (start 108 136.5) (end 108 132.022366) (width 0.3) (layer "F.Cu") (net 2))
 (segment (start 244.25 129.25) (end 235.5 129.25) (width 0.3) (layer "F.Cu") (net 2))
 (segment (start 257.54 131.21) (end 246.21 131.21) (width 0.3) (layer "F.Cu") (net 2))
 (segment (start 275.912 124.086) (end 264.664 124.086) (width 0.3) (layer "F.Cu") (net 2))
 (segment (start 302.43 112.091) (end 279.571 112.091) (width 0.3) (layer "F.Cu") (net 2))
 (segment (start 334.293 103.492) (end 330.785 107) (width 0.3) (layer "F.Cu") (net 2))
 (segment (start 246.21 207.381) (end 246.21 176.196) (width 0.3) (layer "F.Cu") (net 2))
 (segment (start 357.008 103.492) (end 337.75 103.492) (width 0.3) (layer "F.Cu") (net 2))
 (segment (start 124.077 191.611) (end 191.228 124.46) (width 0.3) (layer "F.Cu") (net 2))
 (via (at 244.25 129.25) (size 0.7) (drill 0.3) (layers "F.Cu" "B.Cu") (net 2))
 (segment (start 248.92 129.3) (end 244.3 129.3) (width 0.3) (layer "B.Cu") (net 2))
 (segment (start 244.3 129.3) (end 244.25 129.25) (width 0.3) (layer "B.Cu") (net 2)))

